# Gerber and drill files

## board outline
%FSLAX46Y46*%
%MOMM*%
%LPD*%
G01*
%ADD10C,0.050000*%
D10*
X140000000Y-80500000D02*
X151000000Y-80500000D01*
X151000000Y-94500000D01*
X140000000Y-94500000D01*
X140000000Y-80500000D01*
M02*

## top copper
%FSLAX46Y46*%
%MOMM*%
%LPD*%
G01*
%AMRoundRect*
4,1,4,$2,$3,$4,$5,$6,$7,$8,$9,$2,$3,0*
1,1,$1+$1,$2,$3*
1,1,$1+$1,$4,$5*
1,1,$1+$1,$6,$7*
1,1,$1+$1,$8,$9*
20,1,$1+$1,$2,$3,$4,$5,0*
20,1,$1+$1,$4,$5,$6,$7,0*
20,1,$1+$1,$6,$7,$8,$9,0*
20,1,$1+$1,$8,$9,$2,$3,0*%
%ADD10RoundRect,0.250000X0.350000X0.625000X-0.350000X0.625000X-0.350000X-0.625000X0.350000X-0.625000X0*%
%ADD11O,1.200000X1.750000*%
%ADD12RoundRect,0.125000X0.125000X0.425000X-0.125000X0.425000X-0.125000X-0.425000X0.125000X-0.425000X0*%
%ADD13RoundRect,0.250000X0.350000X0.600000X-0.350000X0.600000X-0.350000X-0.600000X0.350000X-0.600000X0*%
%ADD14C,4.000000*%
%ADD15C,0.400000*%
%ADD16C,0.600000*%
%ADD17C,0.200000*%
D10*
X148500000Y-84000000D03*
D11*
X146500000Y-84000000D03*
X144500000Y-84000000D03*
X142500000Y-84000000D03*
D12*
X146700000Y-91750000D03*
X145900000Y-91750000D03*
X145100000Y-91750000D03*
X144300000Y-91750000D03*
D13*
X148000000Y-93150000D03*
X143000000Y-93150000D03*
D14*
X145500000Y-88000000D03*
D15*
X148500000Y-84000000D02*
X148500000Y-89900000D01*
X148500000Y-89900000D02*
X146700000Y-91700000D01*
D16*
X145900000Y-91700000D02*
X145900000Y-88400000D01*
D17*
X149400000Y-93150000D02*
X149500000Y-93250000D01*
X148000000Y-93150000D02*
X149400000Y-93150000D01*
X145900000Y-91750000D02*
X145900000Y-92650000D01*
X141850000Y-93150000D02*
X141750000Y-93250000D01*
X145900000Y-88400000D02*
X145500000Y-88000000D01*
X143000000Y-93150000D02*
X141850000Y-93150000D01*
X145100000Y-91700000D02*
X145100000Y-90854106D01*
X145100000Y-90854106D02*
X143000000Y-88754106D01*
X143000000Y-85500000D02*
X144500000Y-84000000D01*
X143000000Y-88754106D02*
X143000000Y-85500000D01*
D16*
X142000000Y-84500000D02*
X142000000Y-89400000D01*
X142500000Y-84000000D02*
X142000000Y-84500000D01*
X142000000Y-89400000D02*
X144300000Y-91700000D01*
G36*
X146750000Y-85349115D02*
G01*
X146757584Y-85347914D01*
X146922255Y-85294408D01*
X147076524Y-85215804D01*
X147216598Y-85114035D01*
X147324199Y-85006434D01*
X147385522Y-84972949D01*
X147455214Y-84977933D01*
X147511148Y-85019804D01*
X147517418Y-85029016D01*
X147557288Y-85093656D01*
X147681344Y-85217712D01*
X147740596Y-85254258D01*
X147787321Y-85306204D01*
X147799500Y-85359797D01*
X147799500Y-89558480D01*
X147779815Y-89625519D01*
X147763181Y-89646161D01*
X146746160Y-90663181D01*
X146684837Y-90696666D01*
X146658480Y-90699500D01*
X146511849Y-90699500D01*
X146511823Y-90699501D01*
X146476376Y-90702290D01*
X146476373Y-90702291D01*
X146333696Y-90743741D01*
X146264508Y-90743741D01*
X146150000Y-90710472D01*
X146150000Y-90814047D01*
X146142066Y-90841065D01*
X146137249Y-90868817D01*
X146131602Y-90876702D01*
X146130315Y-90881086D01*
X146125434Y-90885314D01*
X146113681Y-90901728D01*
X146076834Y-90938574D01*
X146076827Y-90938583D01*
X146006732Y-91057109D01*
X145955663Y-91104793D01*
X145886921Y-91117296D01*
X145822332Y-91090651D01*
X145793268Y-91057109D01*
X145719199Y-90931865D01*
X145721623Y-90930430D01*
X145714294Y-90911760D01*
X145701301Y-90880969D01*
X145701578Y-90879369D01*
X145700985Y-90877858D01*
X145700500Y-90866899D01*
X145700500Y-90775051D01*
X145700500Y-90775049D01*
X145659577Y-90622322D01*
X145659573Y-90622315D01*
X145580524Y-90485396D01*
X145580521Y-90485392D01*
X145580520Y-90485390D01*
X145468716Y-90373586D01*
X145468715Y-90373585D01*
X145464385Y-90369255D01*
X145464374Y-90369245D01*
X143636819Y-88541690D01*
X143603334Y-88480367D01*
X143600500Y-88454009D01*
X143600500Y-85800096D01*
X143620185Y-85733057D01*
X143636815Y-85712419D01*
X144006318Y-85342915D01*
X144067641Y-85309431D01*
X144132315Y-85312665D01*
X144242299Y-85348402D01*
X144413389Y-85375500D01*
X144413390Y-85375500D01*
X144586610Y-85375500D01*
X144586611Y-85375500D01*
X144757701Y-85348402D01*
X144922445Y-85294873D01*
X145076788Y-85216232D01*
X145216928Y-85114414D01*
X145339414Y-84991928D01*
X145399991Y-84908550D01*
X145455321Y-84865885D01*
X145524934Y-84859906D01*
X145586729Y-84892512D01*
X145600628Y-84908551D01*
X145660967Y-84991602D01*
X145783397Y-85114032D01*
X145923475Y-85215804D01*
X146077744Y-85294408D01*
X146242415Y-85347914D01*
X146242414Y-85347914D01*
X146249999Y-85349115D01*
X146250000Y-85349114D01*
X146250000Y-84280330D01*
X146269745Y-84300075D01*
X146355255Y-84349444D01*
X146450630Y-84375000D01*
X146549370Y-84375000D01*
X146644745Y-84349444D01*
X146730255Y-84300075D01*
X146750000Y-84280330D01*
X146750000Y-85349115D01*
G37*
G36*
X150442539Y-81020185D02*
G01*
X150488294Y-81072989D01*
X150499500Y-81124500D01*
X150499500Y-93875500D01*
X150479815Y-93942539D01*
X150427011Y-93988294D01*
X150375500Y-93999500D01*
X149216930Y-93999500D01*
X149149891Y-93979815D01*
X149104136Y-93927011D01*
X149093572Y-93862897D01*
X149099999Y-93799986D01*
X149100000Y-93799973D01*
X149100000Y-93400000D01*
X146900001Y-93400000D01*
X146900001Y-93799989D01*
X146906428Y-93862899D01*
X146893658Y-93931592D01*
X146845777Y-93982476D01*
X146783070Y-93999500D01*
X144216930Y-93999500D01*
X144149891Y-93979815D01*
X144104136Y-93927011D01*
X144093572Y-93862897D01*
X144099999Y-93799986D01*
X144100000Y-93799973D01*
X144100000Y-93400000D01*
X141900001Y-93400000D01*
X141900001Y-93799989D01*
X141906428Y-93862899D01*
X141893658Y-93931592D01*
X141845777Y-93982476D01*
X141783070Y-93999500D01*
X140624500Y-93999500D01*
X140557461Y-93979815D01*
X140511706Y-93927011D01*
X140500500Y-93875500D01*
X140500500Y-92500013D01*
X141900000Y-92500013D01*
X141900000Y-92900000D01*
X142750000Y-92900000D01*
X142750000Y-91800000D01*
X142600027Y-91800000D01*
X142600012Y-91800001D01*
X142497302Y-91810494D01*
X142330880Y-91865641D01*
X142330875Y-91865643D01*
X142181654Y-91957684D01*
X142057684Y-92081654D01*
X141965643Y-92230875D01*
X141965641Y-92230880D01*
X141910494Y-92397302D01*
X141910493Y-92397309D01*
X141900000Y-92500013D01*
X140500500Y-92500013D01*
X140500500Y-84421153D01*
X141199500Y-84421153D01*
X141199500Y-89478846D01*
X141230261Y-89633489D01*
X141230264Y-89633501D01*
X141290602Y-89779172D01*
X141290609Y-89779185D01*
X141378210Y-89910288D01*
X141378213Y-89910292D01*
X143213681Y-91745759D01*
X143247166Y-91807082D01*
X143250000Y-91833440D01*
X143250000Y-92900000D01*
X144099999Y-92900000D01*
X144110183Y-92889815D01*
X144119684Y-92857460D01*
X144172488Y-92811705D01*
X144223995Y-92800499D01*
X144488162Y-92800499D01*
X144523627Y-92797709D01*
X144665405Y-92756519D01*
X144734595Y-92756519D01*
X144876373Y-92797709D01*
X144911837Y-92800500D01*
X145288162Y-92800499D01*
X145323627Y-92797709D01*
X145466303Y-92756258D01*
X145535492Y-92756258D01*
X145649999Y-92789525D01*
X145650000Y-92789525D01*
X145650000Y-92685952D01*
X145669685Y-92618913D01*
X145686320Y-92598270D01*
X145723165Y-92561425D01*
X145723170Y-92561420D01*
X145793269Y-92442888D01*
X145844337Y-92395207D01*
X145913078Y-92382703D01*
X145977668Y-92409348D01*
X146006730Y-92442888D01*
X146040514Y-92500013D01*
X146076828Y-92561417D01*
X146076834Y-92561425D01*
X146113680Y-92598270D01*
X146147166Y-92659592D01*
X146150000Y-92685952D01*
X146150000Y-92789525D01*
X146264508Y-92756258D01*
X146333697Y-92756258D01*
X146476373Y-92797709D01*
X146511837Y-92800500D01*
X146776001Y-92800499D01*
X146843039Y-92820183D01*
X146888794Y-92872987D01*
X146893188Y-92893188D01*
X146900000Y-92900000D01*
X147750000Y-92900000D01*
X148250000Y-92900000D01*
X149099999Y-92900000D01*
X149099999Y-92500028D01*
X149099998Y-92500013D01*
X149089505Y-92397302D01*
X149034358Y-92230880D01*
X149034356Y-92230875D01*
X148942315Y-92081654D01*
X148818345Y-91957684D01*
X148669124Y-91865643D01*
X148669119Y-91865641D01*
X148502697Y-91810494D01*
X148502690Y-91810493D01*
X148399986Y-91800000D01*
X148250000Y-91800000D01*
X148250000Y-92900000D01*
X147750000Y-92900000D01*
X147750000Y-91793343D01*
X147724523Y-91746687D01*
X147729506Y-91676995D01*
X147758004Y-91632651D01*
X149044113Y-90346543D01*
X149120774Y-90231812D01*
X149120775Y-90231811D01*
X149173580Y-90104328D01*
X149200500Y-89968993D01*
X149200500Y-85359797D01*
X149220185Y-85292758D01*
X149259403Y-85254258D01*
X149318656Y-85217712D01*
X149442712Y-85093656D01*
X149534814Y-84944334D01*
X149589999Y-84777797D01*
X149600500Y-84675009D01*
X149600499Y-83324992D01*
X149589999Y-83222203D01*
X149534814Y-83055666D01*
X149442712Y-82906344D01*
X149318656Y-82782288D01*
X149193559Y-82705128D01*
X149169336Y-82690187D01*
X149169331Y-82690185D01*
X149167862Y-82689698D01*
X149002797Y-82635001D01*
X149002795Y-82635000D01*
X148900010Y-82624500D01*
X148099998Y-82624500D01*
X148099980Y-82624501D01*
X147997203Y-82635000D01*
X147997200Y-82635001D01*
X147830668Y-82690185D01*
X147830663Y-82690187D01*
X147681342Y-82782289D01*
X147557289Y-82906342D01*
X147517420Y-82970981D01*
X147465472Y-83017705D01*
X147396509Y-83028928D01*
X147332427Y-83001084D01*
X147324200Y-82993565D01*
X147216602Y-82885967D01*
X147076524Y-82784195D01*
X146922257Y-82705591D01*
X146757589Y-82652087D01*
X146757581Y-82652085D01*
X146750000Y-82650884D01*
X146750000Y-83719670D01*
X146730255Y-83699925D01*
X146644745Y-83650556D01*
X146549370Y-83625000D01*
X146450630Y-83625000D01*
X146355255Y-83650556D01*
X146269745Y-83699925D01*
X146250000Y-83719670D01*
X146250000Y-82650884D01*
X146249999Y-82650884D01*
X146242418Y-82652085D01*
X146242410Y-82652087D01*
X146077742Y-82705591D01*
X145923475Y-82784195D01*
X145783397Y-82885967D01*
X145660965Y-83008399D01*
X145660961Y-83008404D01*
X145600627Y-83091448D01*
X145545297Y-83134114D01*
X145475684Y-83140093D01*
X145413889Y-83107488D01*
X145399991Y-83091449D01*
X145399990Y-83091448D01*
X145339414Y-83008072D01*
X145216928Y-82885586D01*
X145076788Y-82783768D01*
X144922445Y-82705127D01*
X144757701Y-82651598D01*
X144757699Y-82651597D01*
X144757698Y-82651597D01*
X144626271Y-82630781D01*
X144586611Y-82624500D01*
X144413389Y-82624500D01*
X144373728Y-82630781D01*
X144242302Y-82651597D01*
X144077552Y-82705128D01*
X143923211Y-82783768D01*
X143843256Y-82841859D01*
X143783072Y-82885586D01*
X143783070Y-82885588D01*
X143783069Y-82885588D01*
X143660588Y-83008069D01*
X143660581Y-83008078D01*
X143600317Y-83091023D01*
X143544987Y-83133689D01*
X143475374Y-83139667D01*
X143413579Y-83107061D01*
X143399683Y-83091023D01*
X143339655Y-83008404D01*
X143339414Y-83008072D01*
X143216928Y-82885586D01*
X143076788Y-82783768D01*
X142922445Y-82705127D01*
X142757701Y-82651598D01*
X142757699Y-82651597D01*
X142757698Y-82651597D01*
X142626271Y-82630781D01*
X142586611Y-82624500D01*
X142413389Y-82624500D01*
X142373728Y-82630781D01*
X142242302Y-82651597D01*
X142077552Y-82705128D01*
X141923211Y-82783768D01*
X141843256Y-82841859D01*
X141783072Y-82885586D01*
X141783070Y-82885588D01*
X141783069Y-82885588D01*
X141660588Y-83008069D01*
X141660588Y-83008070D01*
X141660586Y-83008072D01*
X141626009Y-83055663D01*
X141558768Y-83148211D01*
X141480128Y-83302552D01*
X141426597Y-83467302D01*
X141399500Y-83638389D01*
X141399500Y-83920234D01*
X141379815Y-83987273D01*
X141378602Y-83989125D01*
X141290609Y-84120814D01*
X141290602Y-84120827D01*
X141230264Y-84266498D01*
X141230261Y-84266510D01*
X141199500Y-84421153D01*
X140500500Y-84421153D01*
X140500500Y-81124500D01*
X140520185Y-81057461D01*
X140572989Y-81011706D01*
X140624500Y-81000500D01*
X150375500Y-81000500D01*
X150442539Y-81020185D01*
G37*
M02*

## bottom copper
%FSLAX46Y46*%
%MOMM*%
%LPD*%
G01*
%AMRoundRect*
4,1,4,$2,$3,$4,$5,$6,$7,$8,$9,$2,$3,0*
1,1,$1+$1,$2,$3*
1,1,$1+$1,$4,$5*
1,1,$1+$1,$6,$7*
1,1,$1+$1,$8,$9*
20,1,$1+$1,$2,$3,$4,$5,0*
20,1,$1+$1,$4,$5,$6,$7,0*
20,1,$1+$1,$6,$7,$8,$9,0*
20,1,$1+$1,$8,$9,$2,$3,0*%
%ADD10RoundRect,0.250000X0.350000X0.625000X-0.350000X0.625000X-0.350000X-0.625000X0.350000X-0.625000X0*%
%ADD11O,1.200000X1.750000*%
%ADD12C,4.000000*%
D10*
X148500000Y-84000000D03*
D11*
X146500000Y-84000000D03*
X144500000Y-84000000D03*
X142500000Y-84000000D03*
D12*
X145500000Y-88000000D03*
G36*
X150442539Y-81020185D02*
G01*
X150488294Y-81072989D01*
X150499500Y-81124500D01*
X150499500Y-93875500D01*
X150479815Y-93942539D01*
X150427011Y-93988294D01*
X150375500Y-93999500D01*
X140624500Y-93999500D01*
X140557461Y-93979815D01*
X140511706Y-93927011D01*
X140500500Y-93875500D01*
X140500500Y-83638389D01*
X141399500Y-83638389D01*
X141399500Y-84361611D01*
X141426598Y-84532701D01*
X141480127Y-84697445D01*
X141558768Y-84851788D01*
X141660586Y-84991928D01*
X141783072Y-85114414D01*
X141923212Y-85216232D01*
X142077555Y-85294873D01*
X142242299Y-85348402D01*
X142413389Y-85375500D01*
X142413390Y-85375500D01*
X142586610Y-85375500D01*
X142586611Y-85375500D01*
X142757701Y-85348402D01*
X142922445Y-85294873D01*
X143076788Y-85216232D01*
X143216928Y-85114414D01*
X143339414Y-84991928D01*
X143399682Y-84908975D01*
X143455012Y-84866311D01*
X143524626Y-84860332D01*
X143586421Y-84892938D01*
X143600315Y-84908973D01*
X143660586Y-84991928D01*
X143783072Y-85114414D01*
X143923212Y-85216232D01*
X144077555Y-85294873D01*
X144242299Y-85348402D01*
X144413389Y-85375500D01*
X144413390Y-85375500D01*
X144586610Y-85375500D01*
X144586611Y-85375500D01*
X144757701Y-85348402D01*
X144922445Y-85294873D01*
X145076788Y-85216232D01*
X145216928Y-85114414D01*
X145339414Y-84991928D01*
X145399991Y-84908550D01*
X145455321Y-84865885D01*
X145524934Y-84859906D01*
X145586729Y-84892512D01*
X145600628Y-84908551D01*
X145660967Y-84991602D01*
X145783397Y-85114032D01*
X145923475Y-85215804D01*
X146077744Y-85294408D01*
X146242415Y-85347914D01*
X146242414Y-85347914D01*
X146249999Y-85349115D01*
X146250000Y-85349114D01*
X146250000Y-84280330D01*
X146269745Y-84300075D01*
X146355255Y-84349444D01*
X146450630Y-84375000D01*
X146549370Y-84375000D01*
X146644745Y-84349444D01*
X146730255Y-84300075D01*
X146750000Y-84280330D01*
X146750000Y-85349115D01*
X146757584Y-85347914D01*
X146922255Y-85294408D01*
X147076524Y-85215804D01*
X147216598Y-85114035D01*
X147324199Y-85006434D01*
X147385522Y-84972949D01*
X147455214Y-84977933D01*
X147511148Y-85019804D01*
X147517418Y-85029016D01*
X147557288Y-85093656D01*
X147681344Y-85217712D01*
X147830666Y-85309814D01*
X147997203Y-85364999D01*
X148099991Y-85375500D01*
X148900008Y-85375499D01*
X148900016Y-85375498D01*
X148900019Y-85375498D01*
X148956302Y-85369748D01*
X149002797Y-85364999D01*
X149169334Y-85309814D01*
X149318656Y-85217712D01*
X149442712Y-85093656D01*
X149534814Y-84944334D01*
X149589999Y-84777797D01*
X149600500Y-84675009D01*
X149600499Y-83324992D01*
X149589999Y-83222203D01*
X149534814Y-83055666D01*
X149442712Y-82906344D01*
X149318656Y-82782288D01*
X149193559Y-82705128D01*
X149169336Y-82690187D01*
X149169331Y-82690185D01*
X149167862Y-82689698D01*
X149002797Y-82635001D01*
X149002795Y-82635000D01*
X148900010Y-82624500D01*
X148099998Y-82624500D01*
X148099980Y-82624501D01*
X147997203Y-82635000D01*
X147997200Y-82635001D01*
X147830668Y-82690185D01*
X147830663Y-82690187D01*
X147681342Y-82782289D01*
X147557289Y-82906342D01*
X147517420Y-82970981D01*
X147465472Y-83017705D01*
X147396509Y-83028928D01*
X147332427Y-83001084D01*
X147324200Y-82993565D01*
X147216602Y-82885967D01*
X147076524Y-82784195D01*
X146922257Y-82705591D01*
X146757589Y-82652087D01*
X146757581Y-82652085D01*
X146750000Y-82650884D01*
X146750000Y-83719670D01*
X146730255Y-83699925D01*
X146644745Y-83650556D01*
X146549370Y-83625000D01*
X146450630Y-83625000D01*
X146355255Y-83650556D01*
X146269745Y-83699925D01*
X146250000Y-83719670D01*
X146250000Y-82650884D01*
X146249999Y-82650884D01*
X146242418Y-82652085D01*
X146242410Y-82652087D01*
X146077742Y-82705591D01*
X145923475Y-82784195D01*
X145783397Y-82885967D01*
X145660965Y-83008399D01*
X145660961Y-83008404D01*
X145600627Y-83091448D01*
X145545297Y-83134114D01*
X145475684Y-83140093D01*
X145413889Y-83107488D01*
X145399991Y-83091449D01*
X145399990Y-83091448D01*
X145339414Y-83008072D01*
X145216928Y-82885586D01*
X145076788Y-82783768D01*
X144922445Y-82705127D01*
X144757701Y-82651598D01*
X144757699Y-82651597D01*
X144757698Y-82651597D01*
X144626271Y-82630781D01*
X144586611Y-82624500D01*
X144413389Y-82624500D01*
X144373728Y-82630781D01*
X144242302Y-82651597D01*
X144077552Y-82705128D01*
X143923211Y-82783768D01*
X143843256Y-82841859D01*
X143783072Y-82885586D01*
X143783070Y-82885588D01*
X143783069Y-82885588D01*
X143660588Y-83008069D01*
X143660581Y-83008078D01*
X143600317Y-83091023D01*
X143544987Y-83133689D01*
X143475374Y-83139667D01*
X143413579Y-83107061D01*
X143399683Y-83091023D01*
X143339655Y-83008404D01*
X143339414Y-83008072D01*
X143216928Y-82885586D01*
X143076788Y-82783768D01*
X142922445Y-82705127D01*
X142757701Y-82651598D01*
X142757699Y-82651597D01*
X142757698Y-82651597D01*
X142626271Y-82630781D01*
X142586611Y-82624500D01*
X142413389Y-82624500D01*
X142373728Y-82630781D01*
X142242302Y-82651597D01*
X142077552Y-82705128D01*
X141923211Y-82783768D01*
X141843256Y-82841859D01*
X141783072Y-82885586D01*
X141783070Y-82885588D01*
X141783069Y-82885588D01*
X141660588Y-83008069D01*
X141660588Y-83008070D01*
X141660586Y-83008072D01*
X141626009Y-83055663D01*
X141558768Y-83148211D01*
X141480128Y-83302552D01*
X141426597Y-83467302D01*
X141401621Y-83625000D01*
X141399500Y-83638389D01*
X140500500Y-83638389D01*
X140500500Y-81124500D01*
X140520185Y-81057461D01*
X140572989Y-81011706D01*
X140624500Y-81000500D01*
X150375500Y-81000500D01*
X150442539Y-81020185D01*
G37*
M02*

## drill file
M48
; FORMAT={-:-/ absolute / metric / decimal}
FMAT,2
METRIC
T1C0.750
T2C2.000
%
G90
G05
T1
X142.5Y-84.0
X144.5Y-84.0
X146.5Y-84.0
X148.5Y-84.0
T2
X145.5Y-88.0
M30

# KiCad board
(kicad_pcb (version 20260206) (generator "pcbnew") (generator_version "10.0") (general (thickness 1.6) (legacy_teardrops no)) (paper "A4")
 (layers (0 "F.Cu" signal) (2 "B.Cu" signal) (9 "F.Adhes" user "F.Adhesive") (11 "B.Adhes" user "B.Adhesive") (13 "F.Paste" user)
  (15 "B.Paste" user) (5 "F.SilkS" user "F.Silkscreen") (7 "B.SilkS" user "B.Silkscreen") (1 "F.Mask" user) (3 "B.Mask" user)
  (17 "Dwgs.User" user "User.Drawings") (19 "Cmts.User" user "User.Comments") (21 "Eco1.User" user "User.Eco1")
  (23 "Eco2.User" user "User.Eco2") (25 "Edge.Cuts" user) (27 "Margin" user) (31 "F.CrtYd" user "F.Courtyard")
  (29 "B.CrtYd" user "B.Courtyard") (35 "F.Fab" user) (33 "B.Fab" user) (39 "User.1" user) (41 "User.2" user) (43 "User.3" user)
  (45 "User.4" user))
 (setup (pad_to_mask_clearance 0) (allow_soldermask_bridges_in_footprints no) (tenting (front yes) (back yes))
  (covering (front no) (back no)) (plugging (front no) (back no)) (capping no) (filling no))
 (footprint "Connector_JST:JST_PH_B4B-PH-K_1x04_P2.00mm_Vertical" (layer "F.Cu") (at 148.5 84 180)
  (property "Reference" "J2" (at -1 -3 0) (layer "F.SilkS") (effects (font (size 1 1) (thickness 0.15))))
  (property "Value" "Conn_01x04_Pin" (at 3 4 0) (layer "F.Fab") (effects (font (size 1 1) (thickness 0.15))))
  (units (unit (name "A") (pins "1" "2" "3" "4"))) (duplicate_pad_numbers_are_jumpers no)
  (pad "1" thru_hole roundrect (at 0 0 180) (size 1.2 1.75) (drill 0.75) (layers "*.Cu" "*.Mask") (remove_unused_layers no)
   (roundrect_rratio 0.208333) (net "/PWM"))
  (pad "2" thru_hole oval (at 2 0 180) (size 1.2 1.75) (drill 0.75) (layers "*.Cu" "*.Mask") (remove_unused_layers no) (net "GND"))
  (pad "3" thru_hole oval (at 4 0 180) (size 1.2 1.75) (drill 0.75) (layers "*.Cu" "*.Mask") (remove_unused_layers no) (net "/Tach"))
  (pad "4" thru_hole oval (at 6 0 180) (size 1.2 1.75) (drill 0.75) (layers "*.Cu" "*.Mask") (remove_unused_layers no) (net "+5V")))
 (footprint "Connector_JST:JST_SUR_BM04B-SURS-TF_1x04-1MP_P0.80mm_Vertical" (layer "F.Cu") (at 145.5 92.6 180)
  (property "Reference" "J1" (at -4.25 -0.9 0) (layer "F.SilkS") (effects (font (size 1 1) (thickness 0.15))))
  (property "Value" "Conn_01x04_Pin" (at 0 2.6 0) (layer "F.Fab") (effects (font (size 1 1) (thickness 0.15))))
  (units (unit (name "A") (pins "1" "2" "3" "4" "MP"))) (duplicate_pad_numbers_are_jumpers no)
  (pad "1" smd roundrect (at -1.2 0.85 180) (size 0.5 1.1) (layers "F.Cu" "F.Mask" "F.Paste") (roundrect_rratio 0.25) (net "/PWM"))
  (pad "2" smd roundrect (at -0.4 0.85 180) (size 0.5 1.1) (layers "F.Cu" "F.Mask" "F.Paste") (roundrect_rratio 0.25) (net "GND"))
  (pad "3" smd roundrect (at 0.4 0.85 180) (size 0.5 1.1) (layers "F.Cu" "F.Mask" "F.Paste") (roundrect_rratio 0.25) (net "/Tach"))
  (pad "4" smd roundrect (at 1.2 0.85 180) (size 0.5 1.1) (layers "F.Cu" "F.Mask" "F.Paste") (roundrect_rratio 0.25) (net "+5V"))
  (pad "MP" smd roundrect (at -2.5 -0.55 180) (size 1.2 1.7) (layers "F.Cu" "F.Mask" "F.Paste") (roundrect_rratio 0.208333) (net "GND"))
  (pad "MP" smd roundrect (at 2.5 -0.55 180) (size 1.2 1.7) (layers "F.Cu" "F.Mask" "F.Paste") (roundrect_rratio 0.208333) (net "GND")))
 (gr_rect (start 140 80.5) (end 151 94.5) (stroke (width 0.05) (type default)) (fill no) (layer "Edge.Cuts"))
 (segment (start 148.5 84) (end 148.5 89.9) (width 0.4) (layer "F.Cu") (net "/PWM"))
 (segment (start 148.5 89.9) (end 146.7 91.7) (width 0.4) (layer "F.Cu") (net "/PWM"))
 (segment (start 145.9 91.7) (end 145.9 88.4) (width 0.6) (layer "F.Cu") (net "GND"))
 (segment (start 149.4 93.15) (end 149.5 93.25) (width 0.2) (layer "F.Cu") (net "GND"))
 (segment (start 148 93.15) (end 149.4 93.15) (width 0.2) (layer "F.Cu") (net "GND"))
 (segment (start 145.9 91.75) (end 145.9 92.65) (width 0.2) (layer "F.Cu") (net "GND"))
 (segment (start 141.85 93.15) (end 141.75 93.25) (width 0.2) (layer "F.Cu") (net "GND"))
 (segment (start 145.9 88.4) (end 145.5 88) (width 0.2) (layer "F.Cu") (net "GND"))
 (segment (start 143 93.15) (end 141.85 93.15) (width 0.2) (layer "F.Cu") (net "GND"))
 (via (at 145.5 88) (size 4) (drill 2) (layers "F.Cu" "B.Cu") (free yes) (capping no) (covering (front no) (back no))
  (plugging (front no) (back no)) (filling no) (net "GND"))
 (segment (start 145.1 91.7) (end 145.1 90.854106) (width 0.2) (layer "F.Cu") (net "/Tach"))
 (segment (start 145.1 90.854106) (end 143 88.754106) (width 0.2) (layer "F.Cu") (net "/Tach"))
 (segment (start 143 85.5) (end 144.5 84) (width 0.2) (layer "F.Cu") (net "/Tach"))
 (segment (start 143 88.754106) (end 143 85.5) (width 0.2) (layer "F.Cu") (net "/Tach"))
 (segment (start 142 84.5) (end 142 89.4) (width 0.6) (layer "F.Cu") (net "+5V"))
 (segment (start 142.5 84) (end 142 84.5) (width 0.6) (layer "F.Cu") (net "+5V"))
 (segment (start 142 89.4) (end 144.3 91.7) (width 0.6) (layer "F.Cu") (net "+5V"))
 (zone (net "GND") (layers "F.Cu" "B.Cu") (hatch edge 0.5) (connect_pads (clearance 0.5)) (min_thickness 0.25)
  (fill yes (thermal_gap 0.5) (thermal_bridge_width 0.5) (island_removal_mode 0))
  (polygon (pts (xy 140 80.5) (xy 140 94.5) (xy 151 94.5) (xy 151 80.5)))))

